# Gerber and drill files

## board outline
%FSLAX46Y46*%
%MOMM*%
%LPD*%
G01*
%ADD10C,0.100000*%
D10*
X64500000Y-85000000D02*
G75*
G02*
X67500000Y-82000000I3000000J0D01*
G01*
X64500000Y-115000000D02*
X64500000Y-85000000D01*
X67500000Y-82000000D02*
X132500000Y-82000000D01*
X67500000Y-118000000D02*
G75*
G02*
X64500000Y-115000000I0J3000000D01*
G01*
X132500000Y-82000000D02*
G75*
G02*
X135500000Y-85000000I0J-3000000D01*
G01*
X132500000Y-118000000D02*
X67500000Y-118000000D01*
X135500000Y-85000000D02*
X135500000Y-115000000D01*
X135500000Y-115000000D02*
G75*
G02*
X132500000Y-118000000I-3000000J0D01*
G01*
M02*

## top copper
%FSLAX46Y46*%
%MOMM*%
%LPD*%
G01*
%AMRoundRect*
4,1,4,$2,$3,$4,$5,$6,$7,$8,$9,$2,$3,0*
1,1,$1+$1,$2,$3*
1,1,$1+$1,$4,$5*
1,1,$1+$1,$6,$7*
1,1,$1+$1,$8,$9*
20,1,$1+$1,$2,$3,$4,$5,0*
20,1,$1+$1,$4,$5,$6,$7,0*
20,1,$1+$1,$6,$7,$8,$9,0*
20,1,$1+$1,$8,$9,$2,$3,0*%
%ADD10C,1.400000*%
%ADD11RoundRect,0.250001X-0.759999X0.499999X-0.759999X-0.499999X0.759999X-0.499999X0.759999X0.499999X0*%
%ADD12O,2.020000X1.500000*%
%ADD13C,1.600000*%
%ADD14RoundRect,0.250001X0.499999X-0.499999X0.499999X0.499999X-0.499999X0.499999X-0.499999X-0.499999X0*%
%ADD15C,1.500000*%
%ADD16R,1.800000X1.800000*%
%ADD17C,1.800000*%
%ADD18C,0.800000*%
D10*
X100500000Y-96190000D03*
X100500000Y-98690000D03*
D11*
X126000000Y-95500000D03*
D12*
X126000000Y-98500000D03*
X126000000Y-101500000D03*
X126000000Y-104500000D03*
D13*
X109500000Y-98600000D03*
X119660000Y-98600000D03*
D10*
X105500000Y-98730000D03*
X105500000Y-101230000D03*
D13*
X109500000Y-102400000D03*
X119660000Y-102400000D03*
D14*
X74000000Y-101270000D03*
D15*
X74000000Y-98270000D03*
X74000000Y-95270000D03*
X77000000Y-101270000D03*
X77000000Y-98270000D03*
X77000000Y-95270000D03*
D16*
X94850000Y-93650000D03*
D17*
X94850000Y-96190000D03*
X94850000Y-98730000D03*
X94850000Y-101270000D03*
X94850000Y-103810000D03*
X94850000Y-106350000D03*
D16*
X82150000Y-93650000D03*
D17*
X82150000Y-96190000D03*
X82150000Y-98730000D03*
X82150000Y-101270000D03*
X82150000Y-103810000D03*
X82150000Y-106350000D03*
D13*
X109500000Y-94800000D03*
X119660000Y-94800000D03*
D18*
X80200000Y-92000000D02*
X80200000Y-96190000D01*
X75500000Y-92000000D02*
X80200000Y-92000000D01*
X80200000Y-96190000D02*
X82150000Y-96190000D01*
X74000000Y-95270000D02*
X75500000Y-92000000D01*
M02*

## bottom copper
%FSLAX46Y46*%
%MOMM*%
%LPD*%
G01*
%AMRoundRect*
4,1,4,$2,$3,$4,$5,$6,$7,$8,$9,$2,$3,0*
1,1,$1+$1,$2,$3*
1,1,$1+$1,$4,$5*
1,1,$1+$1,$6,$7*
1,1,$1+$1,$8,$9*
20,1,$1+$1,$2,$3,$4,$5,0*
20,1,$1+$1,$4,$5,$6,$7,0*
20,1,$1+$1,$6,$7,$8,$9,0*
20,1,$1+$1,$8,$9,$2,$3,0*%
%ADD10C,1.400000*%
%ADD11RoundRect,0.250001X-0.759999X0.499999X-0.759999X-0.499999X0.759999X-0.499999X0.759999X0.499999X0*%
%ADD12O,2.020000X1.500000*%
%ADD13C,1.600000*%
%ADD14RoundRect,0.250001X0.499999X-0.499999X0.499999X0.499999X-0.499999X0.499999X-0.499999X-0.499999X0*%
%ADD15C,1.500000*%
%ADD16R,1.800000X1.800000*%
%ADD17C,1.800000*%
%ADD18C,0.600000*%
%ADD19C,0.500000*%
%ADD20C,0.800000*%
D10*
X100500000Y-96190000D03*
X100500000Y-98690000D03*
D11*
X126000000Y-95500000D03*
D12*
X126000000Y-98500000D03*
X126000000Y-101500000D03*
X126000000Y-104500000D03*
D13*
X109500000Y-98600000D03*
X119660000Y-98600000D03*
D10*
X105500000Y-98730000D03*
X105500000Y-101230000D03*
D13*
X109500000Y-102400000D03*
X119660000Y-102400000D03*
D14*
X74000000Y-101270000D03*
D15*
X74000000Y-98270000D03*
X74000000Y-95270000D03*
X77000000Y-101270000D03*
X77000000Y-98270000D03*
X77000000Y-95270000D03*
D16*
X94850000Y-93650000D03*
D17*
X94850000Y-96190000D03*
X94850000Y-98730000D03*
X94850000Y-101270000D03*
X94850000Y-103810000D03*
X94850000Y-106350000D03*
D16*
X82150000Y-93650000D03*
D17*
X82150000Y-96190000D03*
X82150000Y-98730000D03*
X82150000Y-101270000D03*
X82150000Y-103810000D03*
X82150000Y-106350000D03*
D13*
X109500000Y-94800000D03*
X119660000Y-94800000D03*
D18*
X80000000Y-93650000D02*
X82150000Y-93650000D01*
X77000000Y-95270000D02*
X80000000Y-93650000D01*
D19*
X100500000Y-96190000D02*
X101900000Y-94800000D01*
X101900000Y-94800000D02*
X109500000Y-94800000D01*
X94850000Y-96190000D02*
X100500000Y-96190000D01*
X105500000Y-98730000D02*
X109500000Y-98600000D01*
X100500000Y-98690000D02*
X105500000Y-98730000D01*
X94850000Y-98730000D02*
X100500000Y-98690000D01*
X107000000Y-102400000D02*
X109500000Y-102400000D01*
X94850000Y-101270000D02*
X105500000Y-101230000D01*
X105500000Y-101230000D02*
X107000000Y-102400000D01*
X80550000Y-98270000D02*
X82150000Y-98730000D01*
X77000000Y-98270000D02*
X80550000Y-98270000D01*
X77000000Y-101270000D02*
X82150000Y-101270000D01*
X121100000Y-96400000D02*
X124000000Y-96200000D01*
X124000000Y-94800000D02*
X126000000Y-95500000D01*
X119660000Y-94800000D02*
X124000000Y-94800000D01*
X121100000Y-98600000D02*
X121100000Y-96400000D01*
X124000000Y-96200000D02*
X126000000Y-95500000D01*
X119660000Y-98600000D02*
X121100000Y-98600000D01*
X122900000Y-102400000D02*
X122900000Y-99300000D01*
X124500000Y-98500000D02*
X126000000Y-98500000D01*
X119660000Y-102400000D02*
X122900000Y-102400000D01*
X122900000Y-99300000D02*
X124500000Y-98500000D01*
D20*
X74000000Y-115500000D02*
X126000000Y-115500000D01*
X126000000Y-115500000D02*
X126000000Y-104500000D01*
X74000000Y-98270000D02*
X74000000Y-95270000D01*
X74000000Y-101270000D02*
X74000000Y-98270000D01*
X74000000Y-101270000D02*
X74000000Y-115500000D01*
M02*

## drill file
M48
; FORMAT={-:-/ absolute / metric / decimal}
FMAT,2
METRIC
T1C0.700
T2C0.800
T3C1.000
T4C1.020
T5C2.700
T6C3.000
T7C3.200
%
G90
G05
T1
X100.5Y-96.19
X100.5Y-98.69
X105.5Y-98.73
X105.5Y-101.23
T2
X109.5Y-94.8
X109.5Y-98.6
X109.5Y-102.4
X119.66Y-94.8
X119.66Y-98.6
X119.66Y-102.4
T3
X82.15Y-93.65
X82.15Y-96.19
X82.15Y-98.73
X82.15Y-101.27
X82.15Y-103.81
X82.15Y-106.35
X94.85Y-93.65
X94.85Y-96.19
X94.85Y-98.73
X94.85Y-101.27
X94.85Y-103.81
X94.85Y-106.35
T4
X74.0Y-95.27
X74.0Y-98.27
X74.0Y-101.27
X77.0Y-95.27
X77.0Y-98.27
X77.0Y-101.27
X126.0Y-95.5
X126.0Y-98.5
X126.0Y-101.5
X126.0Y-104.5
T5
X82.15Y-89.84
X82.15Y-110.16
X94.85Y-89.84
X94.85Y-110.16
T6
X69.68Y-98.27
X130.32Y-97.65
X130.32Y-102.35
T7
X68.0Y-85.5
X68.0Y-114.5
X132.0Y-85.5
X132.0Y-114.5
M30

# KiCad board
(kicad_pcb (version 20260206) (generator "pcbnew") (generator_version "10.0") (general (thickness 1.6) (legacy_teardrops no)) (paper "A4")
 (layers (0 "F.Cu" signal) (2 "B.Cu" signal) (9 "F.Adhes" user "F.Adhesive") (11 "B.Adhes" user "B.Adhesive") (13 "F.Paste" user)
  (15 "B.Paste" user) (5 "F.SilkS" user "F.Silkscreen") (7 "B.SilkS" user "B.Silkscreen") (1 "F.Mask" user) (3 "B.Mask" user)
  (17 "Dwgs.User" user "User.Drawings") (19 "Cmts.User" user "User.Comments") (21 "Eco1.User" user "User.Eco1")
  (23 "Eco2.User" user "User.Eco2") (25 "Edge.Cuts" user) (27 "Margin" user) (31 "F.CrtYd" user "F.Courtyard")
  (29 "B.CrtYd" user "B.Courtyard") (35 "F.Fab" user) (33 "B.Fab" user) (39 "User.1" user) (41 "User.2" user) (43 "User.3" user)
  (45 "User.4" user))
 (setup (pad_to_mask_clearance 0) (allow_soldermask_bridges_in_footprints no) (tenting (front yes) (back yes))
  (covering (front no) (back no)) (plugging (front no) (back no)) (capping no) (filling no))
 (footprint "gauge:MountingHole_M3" (layer "F.Cu") (at 132 85.5)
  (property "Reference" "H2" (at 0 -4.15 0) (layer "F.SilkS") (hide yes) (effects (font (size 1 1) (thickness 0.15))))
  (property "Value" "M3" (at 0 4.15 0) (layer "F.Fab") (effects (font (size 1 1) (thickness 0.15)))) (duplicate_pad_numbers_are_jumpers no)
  (pad "" np_thru_hole circle (at 0 0) (size 3.2 3.2) (drill 3.2) (layers "*.Cu" "*.Mask")))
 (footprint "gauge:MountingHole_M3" (layer "F.Cu") (at 132 114.5)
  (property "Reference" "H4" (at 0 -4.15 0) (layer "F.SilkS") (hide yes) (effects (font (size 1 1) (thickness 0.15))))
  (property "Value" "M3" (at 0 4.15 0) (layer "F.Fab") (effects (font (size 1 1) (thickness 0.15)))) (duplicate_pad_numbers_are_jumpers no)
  (pad "" np_thru_hole circle (at 0 0) (size 3.2 3.2) (drill 3.2) (layers "*.Cu" "*.Mask")))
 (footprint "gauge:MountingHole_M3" (layer "F.Cu") (at 68 85.5)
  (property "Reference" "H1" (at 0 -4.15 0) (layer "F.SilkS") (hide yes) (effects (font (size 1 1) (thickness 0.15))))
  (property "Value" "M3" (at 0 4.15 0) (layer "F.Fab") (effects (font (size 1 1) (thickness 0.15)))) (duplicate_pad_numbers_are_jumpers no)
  (pad "" np_thru_hole circle (at 0 0) (size 3.2 3.2) (drill 3.2) (layers "*.Cu" "*.Mask")))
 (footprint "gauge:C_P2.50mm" (layer "F.Cu") (at 100.5 96.19 -90)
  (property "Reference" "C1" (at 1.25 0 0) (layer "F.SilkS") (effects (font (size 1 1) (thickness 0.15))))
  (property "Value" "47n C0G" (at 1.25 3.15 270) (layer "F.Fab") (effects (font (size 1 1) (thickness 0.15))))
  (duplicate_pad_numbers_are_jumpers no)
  (pad "1" thru_hole circle (at 0 0 270) (size 1.4 1.4) (drill 0.7) (layers "*.Cu" "*.Mask") (remove_unused_layers no) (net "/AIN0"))
  (pad "2" thru_hole circle (at 2.5 0 270) (size 1.4 1.4) (drill 0.7) (layers "*.Cu" "*.Mask") (remove_unused_layers no) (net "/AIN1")))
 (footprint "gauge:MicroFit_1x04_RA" (layer "F.Cu") (at 126 95.5 -90)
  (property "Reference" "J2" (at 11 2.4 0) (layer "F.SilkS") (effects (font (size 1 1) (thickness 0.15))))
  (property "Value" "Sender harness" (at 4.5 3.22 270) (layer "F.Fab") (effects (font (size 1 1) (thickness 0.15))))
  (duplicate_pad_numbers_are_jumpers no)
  (pad "" np_thru_hole circle (at 2.15 -4.32 270) (size 3 3) (drill 3) (layers "*.Cu" "*.Mask"))
  (pad "" np_thru_hole circle (at 6.85 -4.32 270) (size 3 3) (drill 3) (layers "*.Cu" "*.Mask"))
  (pad "1" thru_hole roundrect (at 0 0 270) (size 1.5 2.02) (drill 1.02) (layers "*.Cu" "*.Mask") (remove_unused_layers no)
   (roundrect_rratio 0.166667) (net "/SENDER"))
  (pad "2" thru_hole oval (at 3 0 270) (size 1.5 2.02) (drill 1.02) (layers "*.Cu" "*.Mask") (remove_unused_layers no) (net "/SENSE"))
  (pad "3" thru_hole oval (at 6 0 270) (size 1.5 2.02) (drill 1.02) (layers "*.Cu" "*.Mask") (remove_unused_layers no)
   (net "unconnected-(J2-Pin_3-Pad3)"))
  (pad "4" thru_hole oval (at 9 0 270) (size 1.5 2.02) (drill 1.02) (layers "*.Cu" "*.Mask") (remove_unused_layers no) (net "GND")))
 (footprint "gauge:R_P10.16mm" (layer "F.Cu") (at 109.5 98.6)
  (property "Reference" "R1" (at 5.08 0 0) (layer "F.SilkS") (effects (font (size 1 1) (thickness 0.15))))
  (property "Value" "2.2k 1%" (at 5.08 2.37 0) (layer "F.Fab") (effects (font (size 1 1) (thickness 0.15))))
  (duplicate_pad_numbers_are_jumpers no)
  (pad "1" thru_hole circle (at 0 0) (size 1.6 1.6) (drill 0.8) (layers "*.Cu" "*.Mask") (remove_unused_layers no) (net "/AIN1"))
  (pad "2" thru_hole circle (at 10.16 0) (size 1.6 1.6) (drill 0.8) (layers "*.Cu" "*.Mask") (remove_unused_layers no) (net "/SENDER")))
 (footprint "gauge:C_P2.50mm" (layer "F.Cu") (at 105.5 98.73 -90)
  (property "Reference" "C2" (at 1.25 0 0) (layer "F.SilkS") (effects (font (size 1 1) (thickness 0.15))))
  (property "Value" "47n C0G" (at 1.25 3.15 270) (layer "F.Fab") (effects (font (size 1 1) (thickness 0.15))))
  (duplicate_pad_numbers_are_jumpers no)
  (pad "1" thru_hole circle (at 0 0 270) (size 1.4 1.4) (drill 0.7) (layers "*.Cu" "*.Mask") (remove_unused_layers no) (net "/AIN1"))
  (pad "2" thru_hole circle (at 2.5 0 270) (size 1.4 1.4) (drill 0.7) (layers "*.Cu" "*.Mask") (remove_unused_layers no) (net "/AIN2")))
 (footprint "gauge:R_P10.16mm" (layer "F.Cu") (at 109.5 102.4)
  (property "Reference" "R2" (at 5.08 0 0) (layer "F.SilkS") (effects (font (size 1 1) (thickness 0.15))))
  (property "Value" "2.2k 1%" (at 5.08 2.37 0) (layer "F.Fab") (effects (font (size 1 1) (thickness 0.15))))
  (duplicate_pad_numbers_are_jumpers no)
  (pad "1" thru_hole circle (at 0 0) (size 1.6 1.6) (drill 0.8) (layers "*.Cu" "*.Mask") (remove_unused_layers no) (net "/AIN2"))
  (pad "2" thru_hole circle (at 10.16 0) (size 1.6 1.6) (drill 0.8) (layers "*.Cu" "*.Mask") (remove_unused_layers no) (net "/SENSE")))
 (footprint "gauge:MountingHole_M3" (layer "F.Cu") (at 68 114.5)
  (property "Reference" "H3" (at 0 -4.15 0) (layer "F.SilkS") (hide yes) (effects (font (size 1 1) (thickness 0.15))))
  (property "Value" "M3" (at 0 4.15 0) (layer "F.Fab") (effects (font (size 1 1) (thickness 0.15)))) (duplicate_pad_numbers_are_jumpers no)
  (pad "" np_thru_hole circle (at 0 0) (size 3.2 3.2) (drill 3.2) (layers "*.Cu" "*.Mask")))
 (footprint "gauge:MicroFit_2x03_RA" (layer "F.Cu") (at 74 101.27 90)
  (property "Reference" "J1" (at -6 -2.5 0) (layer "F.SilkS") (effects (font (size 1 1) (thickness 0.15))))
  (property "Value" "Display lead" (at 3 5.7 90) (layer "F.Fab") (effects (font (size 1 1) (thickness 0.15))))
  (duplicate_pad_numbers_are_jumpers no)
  (pad "" np_thru_hole circle (at 3 -4.32 90) (size 3 3) (drill 3) (layers "*.Cu" "*.Mask"))
  (pad "1" thru_hole roundrect (at 0 0 90) (size 1.5 1.5) (drill 1.02) (layers "*.Cu" "*.Mask") (remove_unused_layers no)
   (roundrect_rratio 0.166667) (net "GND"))
  (pad "2" thru_hole circle (at 3 0 90) (size 1.5 1.5) (drill 1.02) (layers "*.Cu" "*.Mask") (remove_unused_layers no) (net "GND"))
  (pad "3" thru_hole circle (at 6 0 90) (size 1.5 1.5) (drill 1.02) (layers "*.Cu" "*.Mask") (remove_unused_layers no) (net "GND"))
  (pad "4" thru_hole circle (at 0 3 90) (size 1.5 1.5) (drill 1.02) (layers "*.Cu" "*.Mask") (remove_unused_layers no) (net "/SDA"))
  (pad "5" thru_hole circle (at 3 3 90) (size 1.5 1.5) (drill 1.02) (layers "*.Cu" "*.Mask") (remove_unused_layers no) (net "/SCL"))
  (pad "6" thru_hole circle (at 6 3 90) (size 1.5 1.5) (drill 1.02) (layers "*.Cu" "*.Mask") (remove_unused_layers no) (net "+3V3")))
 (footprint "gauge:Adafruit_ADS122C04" (layer "F.Cu") (at 88.5 100 -90)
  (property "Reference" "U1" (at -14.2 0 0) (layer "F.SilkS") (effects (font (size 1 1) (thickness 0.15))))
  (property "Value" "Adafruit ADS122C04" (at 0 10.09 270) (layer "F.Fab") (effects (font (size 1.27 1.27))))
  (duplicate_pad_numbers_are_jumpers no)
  (pad "" np_thru_hole circle (at -10.16 -6.35 270) (size 2.7 2.7) (drill 2.7) (layers "*.Cu"))
  (pad "" np_thru_hole circle (at -10.16 6.35 270) (size 2.7 2.7) (drill 2.7) (layers "*.Cu"))
  (pad "" np_thru_hole circle (at 10.16 -6.35 270) (size 2.7 2.7) (drill 2.7) (layers "*.Cu"))
  (pad "" np_thru_hole circle (at 10.16 6.35 270) (size 2.7 2.7) (drill 2.7) (layers "*.Cu"))
  (pad "1" thru_hole rect (at -6.35 -6.35 270) (size 1.8 1.8) (drill 1) (layers "*.Cu" "*.Mask") (remove_unused_layers no)
   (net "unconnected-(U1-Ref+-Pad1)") (thermal_bridge_angle 45))
  (pad "2" thru_hole circle (at -3.81 -6.35 270) (size 1.8 1.8) (drill 1) (layers "*.Cu" "*.Mask") (remove_unused_layers no) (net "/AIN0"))
  (pad "3" thru_hole circle (at -1.27 -6.35 270) (size 1.8 1.8) (drill 1) (layers "*.Cu" "*.Mask") (remove_unused_layers no) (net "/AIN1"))
  (pad "4" thru_hole circle (at 1.27 -6.35 270) (size 1.8 1.8) (drill 1) (layers "*.Cu" "*.Mask") (remove_unused_layers no) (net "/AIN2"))
  (pad "5" thru_hole circle (at 3.81 -6.35 270) (size 1.8 1.8) (drill 1) (layers "*.Cu" "*.Mask") (remove_unused_layers no)
   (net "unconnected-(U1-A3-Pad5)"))
  (pad "6" thru_hole circle (at 6.35 -6.35 270) (size 1.8 1.8) (drill 1) (layers "*.Cu" "*.Mask") (remove_unused_layers no)
   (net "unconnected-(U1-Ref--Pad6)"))
  (pad "7" thru_hole rect (at -6.35 6.35 270) (size 1.8 1.8) (drill 1) (layers "*.Cu" "*.Mask") (remove_unused_layers no) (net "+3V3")
   (thermal_bridge_angle 45))
  (pad "8" thru_hole circle (at -3.81 6.35 270) (size 1.8 1.8) (drill 1) (layers "*.Cu" "*.Mask") (remove_unused_layers no) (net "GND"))
  (pad "9" thru_hole circle (at -1.27 6.35 270) (size 1.8 1.8) (drill 1) (layers "*.Cu" "*.Mask") (remove_unused_layers no) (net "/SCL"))
  (pad "10" thru_hole circle (at 1.27 6.35 270) (size 1.8 1.8) (drill 1) (layers "*.Cu" "*.Mask") (remove_unused_layers no) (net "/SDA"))
  (pad "11" thru_hole circle (at 3.81 6.35 270) (size 1.8 1.8) (drill 1) (layers "*.Cu" "*.Mask") (remove_unused_layers no)
   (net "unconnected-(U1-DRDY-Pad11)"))
  (pad "12" thru_hole circle (at 6.35 6.35 270) (size 1.8 1.8) (drill 1) (layers "*.Cu" "*.Mask") (remove_unused_layers no)
   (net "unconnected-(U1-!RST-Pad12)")))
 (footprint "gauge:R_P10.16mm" (layer "F.Cu") (at 109.5 94.8)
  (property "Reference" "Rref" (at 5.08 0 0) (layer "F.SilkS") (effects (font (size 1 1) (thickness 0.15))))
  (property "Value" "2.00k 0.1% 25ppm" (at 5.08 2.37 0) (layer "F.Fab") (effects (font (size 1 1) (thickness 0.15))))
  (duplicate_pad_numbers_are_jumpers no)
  (pad "1" thru_hole circle (at 0 0) (size 1.6 1.6) (drill 0.8) (layers "*.Cu" "*.Mask") (remove_unused_layers no) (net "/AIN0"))
  (pad "2" thru_hole circle (at 10.16 0) (size 1.6 1.6) (drill 0.8) (layers "*.Cu" "*.Mask") (remove_unused_layers no) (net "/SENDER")))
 (gr_arc (start 64.5 85) (mid 65.37868 82.87868) (end 67.5 82) (stroke (width 0.1) (type default)) (layer "Edge.Cuts"))
 (gr_line (start 64.5 115) (end 64.5 85) (stroke (width 0.1) (type default)) (layer "Edge.Cuts"))
 (gr_line (start 67.5 82) (end 132.5 82) (stroke (width 0.1) (type default)) (layer "Edge.Cuts"))
 (gr_arc (start 67.5 118) (mid 65.37868 117.12132) (end 64.5 115) (stroke (width 0.1) (type default)) (layer "Edge.Cuts"))
 (gr_arc (start 132.5 82) (mid 134.62132 82.87868) (end 135.5 85) (stroke (width 0.1) (type default)) (layer "Edge.Cuts"))
 (gr_line (start 132.5 118) (end 67.5 118) (stroke (width 0.1) (type default)) (layer "Edge.Cuts"))
 (gr_line (start 135.5 85) (end 135.5 115) (stroke (width 0.1) (type default)) (layer "Edge.Cuts"))
 (gr_arc (start 135.5 115) (mid 134.62132 117.12132) (end 132.5 118) (stroke (width 0.1) (type default)) (layer "Edge.Cuts"))
 (segment (start 80 93.65) (end 82.15 93.65) (width 0.6) (layer "B.Cu") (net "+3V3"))
 (segment (start 77 95.27) (end 80 93.65) (width 0.6) (layer "B.Cu") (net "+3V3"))
 (segment (start 100.5 96.19) (end 101.9 94.8) (width 0.5) (layer "B.Cu") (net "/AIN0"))
 (segment (start 101.9 94.8) (end 109.5 94.8) (width 0.5) (layer "B.Cu") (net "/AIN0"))
 (segment (start 94.85 96.19) (end 100.5 96.19) (width 0.5) (layer "B.Cu") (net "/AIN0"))
 (segment (start 105.5 98.73) (end 109.5 98.6) (width 0.5) (layer "B.Cu") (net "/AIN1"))
 (segment (start 100.5 98.69) (end 105.5 98.73) (width 0.5) (layer "B.Cu") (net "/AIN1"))
 (segment (start 94.85 98.73) (end 100.5 98.69) (width 0.5) (layer "B.Cu") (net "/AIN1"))
 (segment (start 107 102.4) (end 109.5 102.4) (width 0.5) (layer "B.Cu") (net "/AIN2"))
 (segment (start 94.85 101.27) (end 105.5 101.23) (width 0.5) (layer "B.Cu") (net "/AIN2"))
 (segment (start 105.5 101.23) (end 107 102.4) (width 0.5) (layer "B.Cu") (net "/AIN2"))
 (segment (start 80.55 98.27) (end 82.15 98.73) (width 0.5) (layer "B.Cu") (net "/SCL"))
 (segment (start 77 98.27) (end 80.55 98.27) (width 0.5) (layer "B.Cu") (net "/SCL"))
 (segment (start 77 101.27) (end 82.15 101.27) (width 0.5) (layer "B.Cu") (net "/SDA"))
 (segment (start 121.1 96.4) (end 124 96.2) (width 0.5) (layer "B.Cu") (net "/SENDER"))
 (segment (start 124 94.8) (end 126 95.5) (width 0.5) (layer "B.Cu") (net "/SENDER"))
 (segment (start 119.66 94.8) (end 124 94.8) (width 0.5) (layer "B.Cu") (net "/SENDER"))
 (segment (start 121.1 98.6) (end 121.1 96.4) (width 0.5) (layer "B.Cu") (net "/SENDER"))
 (segment (start 124 96.2) (end 126 95.5) (width 0.5) (layer "B.Cu") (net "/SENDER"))
 (segment (start 119.66 98.6) (end 121.1 98.6) (width 0.5) (layer "B.Cu") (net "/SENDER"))
 (segment (start 122.9 102.4) (end 122.9 99.3) (width 0.5) (layer "B.Cu") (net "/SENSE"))
 (segment (start 124.5 98.5) (end 126 98.5) (width 0.5) (layer "B.Cu") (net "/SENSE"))
 (segment (start 119.66 102.4) (end 122.9 102.4) (width 0.5) (layer "B.Cu") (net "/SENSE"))
 (segment (start 122.9 99.3) (end 124.5 98.5) (width 0.5) (layer "B.Cu") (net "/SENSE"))
 (segment (start 80.2 92) (end 80.2 96.19) (width 0.8) (layer "F.Cu") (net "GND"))
 (segment (start 75.5 92) (end 80.2 92) (width 0.8) (layer "F.Cu") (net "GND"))
 (segment (start 80.2 96.19) (end 82.15 96.19) (width 0.8) (layer "F.Cu") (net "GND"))
 (segment (start 74 95.27) (end 75.5 92) (width 0.8) (layer "F.Cu") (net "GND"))
 (segment (start 74 115.5) (end 126 115.5) (width 0.8) (layer "B.Cu") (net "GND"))
 (segment (start 126 115.5) (end 126 104.5) (width 0.8) (layer "B.Cu") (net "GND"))
 (segment (start 74 98.27) (end 74 95.27) (width 0.8) (layer "B.Cu") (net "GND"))
 (segment (start 74 101.27) (end 74 98.27) (width 0.8) (layer "B.Cu") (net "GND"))
 (segment (start 74 101.27) (end 74 115.5) (width 0.8) (layer "B.Cu") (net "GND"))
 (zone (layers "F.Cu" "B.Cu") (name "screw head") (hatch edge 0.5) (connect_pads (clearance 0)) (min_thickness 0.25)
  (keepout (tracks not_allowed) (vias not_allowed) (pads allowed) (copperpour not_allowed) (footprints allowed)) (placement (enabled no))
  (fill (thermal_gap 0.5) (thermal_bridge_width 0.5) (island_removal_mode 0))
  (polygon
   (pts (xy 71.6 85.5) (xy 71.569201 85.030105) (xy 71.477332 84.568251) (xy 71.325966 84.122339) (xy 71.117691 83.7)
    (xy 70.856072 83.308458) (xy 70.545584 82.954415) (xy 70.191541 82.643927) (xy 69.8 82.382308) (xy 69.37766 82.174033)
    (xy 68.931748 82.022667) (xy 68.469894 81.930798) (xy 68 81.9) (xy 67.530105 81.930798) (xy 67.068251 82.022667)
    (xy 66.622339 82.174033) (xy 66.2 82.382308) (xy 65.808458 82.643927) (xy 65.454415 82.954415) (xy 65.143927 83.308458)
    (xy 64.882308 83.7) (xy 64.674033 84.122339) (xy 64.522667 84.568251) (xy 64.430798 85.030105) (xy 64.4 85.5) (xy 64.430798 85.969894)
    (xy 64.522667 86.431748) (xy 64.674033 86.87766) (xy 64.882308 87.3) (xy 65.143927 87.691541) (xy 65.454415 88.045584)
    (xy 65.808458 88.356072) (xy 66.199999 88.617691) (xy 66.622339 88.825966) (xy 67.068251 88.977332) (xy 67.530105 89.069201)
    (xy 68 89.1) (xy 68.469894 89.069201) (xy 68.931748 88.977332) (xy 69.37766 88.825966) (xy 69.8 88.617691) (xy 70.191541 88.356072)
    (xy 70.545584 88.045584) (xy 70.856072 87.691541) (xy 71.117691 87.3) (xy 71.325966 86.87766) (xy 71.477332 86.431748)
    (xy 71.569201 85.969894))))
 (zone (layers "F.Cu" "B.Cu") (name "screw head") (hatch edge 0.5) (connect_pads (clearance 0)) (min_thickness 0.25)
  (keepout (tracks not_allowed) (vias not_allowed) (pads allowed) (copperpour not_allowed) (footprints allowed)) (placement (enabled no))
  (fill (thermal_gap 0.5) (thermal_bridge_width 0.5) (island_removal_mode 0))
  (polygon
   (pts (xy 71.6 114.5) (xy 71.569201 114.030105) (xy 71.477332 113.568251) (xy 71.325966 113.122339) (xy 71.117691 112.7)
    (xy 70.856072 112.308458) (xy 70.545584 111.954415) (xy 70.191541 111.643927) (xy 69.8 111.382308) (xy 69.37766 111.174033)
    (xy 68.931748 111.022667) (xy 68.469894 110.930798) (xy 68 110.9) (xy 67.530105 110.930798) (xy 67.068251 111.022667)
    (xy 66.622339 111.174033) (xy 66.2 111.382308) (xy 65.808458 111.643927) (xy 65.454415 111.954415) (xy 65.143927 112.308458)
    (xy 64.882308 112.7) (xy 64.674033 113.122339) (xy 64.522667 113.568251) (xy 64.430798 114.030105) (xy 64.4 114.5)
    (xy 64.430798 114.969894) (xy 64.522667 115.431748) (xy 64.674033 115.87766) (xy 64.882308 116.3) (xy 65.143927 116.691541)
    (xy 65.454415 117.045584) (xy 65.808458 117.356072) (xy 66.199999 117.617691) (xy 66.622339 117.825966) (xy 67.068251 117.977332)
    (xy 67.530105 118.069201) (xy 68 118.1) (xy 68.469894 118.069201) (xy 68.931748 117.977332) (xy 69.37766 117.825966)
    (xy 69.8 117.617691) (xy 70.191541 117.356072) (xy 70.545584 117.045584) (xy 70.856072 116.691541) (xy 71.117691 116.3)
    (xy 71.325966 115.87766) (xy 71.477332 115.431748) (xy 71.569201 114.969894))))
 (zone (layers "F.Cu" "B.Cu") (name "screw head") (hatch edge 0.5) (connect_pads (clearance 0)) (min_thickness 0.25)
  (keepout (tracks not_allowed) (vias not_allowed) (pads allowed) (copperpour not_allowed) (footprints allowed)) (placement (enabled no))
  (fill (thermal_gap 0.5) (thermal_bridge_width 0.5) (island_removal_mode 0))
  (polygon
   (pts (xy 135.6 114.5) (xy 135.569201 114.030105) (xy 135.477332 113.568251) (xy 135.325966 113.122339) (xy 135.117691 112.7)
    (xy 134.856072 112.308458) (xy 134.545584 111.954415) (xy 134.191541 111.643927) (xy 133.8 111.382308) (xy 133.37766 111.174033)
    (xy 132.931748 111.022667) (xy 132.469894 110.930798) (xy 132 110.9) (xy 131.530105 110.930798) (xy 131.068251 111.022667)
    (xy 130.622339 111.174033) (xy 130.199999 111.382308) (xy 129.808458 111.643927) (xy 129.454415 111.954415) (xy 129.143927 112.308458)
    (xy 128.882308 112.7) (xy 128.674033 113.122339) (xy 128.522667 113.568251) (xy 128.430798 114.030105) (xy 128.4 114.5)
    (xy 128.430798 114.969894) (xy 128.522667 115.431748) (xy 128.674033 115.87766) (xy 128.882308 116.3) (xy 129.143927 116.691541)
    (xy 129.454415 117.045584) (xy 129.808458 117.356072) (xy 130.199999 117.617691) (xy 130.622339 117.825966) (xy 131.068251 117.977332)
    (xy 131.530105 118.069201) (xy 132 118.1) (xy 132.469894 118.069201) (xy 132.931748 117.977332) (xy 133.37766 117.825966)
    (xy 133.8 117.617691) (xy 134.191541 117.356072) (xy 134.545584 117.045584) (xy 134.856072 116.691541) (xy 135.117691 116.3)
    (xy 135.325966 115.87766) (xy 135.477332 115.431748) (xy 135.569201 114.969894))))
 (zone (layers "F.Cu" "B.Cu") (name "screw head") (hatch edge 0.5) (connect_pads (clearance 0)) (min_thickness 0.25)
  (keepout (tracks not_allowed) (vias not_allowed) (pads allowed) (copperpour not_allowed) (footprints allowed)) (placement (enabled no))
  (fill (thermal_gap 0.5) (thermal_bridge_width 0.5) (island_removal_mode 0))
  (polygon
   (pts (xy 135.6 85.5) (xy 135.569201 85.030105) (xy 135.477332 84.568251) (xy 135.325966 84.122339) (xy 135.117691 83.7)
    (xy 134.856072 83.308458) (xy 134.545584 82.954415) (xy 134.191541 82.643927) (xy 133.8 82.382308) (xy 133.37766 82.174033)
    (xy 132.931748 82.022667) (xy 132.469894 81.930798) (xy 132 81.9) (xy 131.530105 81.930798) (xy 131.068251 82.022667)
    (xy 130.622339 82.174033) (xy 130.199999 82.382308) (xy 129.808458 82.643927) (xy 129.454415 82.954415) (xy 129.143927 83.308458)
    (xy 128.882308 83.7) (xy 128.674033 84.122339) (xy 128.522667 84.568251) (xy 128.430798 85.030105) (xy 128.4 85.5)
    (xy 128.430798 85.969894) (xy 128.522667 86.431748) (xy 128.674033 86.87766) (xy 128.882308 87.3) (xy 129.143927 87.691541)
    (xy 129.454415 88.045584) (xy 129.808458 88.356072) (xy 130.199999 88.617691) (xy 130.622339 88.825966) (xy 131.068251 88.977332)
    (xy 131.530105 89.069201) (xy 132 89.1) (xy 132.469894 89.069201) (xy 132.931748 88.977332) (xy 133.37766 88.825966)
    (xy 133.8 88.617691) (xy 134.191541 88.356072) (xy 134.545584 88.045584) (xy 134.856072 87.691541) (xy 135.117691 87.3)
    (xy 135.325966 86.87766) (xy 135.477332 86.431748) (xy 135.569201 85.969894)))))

